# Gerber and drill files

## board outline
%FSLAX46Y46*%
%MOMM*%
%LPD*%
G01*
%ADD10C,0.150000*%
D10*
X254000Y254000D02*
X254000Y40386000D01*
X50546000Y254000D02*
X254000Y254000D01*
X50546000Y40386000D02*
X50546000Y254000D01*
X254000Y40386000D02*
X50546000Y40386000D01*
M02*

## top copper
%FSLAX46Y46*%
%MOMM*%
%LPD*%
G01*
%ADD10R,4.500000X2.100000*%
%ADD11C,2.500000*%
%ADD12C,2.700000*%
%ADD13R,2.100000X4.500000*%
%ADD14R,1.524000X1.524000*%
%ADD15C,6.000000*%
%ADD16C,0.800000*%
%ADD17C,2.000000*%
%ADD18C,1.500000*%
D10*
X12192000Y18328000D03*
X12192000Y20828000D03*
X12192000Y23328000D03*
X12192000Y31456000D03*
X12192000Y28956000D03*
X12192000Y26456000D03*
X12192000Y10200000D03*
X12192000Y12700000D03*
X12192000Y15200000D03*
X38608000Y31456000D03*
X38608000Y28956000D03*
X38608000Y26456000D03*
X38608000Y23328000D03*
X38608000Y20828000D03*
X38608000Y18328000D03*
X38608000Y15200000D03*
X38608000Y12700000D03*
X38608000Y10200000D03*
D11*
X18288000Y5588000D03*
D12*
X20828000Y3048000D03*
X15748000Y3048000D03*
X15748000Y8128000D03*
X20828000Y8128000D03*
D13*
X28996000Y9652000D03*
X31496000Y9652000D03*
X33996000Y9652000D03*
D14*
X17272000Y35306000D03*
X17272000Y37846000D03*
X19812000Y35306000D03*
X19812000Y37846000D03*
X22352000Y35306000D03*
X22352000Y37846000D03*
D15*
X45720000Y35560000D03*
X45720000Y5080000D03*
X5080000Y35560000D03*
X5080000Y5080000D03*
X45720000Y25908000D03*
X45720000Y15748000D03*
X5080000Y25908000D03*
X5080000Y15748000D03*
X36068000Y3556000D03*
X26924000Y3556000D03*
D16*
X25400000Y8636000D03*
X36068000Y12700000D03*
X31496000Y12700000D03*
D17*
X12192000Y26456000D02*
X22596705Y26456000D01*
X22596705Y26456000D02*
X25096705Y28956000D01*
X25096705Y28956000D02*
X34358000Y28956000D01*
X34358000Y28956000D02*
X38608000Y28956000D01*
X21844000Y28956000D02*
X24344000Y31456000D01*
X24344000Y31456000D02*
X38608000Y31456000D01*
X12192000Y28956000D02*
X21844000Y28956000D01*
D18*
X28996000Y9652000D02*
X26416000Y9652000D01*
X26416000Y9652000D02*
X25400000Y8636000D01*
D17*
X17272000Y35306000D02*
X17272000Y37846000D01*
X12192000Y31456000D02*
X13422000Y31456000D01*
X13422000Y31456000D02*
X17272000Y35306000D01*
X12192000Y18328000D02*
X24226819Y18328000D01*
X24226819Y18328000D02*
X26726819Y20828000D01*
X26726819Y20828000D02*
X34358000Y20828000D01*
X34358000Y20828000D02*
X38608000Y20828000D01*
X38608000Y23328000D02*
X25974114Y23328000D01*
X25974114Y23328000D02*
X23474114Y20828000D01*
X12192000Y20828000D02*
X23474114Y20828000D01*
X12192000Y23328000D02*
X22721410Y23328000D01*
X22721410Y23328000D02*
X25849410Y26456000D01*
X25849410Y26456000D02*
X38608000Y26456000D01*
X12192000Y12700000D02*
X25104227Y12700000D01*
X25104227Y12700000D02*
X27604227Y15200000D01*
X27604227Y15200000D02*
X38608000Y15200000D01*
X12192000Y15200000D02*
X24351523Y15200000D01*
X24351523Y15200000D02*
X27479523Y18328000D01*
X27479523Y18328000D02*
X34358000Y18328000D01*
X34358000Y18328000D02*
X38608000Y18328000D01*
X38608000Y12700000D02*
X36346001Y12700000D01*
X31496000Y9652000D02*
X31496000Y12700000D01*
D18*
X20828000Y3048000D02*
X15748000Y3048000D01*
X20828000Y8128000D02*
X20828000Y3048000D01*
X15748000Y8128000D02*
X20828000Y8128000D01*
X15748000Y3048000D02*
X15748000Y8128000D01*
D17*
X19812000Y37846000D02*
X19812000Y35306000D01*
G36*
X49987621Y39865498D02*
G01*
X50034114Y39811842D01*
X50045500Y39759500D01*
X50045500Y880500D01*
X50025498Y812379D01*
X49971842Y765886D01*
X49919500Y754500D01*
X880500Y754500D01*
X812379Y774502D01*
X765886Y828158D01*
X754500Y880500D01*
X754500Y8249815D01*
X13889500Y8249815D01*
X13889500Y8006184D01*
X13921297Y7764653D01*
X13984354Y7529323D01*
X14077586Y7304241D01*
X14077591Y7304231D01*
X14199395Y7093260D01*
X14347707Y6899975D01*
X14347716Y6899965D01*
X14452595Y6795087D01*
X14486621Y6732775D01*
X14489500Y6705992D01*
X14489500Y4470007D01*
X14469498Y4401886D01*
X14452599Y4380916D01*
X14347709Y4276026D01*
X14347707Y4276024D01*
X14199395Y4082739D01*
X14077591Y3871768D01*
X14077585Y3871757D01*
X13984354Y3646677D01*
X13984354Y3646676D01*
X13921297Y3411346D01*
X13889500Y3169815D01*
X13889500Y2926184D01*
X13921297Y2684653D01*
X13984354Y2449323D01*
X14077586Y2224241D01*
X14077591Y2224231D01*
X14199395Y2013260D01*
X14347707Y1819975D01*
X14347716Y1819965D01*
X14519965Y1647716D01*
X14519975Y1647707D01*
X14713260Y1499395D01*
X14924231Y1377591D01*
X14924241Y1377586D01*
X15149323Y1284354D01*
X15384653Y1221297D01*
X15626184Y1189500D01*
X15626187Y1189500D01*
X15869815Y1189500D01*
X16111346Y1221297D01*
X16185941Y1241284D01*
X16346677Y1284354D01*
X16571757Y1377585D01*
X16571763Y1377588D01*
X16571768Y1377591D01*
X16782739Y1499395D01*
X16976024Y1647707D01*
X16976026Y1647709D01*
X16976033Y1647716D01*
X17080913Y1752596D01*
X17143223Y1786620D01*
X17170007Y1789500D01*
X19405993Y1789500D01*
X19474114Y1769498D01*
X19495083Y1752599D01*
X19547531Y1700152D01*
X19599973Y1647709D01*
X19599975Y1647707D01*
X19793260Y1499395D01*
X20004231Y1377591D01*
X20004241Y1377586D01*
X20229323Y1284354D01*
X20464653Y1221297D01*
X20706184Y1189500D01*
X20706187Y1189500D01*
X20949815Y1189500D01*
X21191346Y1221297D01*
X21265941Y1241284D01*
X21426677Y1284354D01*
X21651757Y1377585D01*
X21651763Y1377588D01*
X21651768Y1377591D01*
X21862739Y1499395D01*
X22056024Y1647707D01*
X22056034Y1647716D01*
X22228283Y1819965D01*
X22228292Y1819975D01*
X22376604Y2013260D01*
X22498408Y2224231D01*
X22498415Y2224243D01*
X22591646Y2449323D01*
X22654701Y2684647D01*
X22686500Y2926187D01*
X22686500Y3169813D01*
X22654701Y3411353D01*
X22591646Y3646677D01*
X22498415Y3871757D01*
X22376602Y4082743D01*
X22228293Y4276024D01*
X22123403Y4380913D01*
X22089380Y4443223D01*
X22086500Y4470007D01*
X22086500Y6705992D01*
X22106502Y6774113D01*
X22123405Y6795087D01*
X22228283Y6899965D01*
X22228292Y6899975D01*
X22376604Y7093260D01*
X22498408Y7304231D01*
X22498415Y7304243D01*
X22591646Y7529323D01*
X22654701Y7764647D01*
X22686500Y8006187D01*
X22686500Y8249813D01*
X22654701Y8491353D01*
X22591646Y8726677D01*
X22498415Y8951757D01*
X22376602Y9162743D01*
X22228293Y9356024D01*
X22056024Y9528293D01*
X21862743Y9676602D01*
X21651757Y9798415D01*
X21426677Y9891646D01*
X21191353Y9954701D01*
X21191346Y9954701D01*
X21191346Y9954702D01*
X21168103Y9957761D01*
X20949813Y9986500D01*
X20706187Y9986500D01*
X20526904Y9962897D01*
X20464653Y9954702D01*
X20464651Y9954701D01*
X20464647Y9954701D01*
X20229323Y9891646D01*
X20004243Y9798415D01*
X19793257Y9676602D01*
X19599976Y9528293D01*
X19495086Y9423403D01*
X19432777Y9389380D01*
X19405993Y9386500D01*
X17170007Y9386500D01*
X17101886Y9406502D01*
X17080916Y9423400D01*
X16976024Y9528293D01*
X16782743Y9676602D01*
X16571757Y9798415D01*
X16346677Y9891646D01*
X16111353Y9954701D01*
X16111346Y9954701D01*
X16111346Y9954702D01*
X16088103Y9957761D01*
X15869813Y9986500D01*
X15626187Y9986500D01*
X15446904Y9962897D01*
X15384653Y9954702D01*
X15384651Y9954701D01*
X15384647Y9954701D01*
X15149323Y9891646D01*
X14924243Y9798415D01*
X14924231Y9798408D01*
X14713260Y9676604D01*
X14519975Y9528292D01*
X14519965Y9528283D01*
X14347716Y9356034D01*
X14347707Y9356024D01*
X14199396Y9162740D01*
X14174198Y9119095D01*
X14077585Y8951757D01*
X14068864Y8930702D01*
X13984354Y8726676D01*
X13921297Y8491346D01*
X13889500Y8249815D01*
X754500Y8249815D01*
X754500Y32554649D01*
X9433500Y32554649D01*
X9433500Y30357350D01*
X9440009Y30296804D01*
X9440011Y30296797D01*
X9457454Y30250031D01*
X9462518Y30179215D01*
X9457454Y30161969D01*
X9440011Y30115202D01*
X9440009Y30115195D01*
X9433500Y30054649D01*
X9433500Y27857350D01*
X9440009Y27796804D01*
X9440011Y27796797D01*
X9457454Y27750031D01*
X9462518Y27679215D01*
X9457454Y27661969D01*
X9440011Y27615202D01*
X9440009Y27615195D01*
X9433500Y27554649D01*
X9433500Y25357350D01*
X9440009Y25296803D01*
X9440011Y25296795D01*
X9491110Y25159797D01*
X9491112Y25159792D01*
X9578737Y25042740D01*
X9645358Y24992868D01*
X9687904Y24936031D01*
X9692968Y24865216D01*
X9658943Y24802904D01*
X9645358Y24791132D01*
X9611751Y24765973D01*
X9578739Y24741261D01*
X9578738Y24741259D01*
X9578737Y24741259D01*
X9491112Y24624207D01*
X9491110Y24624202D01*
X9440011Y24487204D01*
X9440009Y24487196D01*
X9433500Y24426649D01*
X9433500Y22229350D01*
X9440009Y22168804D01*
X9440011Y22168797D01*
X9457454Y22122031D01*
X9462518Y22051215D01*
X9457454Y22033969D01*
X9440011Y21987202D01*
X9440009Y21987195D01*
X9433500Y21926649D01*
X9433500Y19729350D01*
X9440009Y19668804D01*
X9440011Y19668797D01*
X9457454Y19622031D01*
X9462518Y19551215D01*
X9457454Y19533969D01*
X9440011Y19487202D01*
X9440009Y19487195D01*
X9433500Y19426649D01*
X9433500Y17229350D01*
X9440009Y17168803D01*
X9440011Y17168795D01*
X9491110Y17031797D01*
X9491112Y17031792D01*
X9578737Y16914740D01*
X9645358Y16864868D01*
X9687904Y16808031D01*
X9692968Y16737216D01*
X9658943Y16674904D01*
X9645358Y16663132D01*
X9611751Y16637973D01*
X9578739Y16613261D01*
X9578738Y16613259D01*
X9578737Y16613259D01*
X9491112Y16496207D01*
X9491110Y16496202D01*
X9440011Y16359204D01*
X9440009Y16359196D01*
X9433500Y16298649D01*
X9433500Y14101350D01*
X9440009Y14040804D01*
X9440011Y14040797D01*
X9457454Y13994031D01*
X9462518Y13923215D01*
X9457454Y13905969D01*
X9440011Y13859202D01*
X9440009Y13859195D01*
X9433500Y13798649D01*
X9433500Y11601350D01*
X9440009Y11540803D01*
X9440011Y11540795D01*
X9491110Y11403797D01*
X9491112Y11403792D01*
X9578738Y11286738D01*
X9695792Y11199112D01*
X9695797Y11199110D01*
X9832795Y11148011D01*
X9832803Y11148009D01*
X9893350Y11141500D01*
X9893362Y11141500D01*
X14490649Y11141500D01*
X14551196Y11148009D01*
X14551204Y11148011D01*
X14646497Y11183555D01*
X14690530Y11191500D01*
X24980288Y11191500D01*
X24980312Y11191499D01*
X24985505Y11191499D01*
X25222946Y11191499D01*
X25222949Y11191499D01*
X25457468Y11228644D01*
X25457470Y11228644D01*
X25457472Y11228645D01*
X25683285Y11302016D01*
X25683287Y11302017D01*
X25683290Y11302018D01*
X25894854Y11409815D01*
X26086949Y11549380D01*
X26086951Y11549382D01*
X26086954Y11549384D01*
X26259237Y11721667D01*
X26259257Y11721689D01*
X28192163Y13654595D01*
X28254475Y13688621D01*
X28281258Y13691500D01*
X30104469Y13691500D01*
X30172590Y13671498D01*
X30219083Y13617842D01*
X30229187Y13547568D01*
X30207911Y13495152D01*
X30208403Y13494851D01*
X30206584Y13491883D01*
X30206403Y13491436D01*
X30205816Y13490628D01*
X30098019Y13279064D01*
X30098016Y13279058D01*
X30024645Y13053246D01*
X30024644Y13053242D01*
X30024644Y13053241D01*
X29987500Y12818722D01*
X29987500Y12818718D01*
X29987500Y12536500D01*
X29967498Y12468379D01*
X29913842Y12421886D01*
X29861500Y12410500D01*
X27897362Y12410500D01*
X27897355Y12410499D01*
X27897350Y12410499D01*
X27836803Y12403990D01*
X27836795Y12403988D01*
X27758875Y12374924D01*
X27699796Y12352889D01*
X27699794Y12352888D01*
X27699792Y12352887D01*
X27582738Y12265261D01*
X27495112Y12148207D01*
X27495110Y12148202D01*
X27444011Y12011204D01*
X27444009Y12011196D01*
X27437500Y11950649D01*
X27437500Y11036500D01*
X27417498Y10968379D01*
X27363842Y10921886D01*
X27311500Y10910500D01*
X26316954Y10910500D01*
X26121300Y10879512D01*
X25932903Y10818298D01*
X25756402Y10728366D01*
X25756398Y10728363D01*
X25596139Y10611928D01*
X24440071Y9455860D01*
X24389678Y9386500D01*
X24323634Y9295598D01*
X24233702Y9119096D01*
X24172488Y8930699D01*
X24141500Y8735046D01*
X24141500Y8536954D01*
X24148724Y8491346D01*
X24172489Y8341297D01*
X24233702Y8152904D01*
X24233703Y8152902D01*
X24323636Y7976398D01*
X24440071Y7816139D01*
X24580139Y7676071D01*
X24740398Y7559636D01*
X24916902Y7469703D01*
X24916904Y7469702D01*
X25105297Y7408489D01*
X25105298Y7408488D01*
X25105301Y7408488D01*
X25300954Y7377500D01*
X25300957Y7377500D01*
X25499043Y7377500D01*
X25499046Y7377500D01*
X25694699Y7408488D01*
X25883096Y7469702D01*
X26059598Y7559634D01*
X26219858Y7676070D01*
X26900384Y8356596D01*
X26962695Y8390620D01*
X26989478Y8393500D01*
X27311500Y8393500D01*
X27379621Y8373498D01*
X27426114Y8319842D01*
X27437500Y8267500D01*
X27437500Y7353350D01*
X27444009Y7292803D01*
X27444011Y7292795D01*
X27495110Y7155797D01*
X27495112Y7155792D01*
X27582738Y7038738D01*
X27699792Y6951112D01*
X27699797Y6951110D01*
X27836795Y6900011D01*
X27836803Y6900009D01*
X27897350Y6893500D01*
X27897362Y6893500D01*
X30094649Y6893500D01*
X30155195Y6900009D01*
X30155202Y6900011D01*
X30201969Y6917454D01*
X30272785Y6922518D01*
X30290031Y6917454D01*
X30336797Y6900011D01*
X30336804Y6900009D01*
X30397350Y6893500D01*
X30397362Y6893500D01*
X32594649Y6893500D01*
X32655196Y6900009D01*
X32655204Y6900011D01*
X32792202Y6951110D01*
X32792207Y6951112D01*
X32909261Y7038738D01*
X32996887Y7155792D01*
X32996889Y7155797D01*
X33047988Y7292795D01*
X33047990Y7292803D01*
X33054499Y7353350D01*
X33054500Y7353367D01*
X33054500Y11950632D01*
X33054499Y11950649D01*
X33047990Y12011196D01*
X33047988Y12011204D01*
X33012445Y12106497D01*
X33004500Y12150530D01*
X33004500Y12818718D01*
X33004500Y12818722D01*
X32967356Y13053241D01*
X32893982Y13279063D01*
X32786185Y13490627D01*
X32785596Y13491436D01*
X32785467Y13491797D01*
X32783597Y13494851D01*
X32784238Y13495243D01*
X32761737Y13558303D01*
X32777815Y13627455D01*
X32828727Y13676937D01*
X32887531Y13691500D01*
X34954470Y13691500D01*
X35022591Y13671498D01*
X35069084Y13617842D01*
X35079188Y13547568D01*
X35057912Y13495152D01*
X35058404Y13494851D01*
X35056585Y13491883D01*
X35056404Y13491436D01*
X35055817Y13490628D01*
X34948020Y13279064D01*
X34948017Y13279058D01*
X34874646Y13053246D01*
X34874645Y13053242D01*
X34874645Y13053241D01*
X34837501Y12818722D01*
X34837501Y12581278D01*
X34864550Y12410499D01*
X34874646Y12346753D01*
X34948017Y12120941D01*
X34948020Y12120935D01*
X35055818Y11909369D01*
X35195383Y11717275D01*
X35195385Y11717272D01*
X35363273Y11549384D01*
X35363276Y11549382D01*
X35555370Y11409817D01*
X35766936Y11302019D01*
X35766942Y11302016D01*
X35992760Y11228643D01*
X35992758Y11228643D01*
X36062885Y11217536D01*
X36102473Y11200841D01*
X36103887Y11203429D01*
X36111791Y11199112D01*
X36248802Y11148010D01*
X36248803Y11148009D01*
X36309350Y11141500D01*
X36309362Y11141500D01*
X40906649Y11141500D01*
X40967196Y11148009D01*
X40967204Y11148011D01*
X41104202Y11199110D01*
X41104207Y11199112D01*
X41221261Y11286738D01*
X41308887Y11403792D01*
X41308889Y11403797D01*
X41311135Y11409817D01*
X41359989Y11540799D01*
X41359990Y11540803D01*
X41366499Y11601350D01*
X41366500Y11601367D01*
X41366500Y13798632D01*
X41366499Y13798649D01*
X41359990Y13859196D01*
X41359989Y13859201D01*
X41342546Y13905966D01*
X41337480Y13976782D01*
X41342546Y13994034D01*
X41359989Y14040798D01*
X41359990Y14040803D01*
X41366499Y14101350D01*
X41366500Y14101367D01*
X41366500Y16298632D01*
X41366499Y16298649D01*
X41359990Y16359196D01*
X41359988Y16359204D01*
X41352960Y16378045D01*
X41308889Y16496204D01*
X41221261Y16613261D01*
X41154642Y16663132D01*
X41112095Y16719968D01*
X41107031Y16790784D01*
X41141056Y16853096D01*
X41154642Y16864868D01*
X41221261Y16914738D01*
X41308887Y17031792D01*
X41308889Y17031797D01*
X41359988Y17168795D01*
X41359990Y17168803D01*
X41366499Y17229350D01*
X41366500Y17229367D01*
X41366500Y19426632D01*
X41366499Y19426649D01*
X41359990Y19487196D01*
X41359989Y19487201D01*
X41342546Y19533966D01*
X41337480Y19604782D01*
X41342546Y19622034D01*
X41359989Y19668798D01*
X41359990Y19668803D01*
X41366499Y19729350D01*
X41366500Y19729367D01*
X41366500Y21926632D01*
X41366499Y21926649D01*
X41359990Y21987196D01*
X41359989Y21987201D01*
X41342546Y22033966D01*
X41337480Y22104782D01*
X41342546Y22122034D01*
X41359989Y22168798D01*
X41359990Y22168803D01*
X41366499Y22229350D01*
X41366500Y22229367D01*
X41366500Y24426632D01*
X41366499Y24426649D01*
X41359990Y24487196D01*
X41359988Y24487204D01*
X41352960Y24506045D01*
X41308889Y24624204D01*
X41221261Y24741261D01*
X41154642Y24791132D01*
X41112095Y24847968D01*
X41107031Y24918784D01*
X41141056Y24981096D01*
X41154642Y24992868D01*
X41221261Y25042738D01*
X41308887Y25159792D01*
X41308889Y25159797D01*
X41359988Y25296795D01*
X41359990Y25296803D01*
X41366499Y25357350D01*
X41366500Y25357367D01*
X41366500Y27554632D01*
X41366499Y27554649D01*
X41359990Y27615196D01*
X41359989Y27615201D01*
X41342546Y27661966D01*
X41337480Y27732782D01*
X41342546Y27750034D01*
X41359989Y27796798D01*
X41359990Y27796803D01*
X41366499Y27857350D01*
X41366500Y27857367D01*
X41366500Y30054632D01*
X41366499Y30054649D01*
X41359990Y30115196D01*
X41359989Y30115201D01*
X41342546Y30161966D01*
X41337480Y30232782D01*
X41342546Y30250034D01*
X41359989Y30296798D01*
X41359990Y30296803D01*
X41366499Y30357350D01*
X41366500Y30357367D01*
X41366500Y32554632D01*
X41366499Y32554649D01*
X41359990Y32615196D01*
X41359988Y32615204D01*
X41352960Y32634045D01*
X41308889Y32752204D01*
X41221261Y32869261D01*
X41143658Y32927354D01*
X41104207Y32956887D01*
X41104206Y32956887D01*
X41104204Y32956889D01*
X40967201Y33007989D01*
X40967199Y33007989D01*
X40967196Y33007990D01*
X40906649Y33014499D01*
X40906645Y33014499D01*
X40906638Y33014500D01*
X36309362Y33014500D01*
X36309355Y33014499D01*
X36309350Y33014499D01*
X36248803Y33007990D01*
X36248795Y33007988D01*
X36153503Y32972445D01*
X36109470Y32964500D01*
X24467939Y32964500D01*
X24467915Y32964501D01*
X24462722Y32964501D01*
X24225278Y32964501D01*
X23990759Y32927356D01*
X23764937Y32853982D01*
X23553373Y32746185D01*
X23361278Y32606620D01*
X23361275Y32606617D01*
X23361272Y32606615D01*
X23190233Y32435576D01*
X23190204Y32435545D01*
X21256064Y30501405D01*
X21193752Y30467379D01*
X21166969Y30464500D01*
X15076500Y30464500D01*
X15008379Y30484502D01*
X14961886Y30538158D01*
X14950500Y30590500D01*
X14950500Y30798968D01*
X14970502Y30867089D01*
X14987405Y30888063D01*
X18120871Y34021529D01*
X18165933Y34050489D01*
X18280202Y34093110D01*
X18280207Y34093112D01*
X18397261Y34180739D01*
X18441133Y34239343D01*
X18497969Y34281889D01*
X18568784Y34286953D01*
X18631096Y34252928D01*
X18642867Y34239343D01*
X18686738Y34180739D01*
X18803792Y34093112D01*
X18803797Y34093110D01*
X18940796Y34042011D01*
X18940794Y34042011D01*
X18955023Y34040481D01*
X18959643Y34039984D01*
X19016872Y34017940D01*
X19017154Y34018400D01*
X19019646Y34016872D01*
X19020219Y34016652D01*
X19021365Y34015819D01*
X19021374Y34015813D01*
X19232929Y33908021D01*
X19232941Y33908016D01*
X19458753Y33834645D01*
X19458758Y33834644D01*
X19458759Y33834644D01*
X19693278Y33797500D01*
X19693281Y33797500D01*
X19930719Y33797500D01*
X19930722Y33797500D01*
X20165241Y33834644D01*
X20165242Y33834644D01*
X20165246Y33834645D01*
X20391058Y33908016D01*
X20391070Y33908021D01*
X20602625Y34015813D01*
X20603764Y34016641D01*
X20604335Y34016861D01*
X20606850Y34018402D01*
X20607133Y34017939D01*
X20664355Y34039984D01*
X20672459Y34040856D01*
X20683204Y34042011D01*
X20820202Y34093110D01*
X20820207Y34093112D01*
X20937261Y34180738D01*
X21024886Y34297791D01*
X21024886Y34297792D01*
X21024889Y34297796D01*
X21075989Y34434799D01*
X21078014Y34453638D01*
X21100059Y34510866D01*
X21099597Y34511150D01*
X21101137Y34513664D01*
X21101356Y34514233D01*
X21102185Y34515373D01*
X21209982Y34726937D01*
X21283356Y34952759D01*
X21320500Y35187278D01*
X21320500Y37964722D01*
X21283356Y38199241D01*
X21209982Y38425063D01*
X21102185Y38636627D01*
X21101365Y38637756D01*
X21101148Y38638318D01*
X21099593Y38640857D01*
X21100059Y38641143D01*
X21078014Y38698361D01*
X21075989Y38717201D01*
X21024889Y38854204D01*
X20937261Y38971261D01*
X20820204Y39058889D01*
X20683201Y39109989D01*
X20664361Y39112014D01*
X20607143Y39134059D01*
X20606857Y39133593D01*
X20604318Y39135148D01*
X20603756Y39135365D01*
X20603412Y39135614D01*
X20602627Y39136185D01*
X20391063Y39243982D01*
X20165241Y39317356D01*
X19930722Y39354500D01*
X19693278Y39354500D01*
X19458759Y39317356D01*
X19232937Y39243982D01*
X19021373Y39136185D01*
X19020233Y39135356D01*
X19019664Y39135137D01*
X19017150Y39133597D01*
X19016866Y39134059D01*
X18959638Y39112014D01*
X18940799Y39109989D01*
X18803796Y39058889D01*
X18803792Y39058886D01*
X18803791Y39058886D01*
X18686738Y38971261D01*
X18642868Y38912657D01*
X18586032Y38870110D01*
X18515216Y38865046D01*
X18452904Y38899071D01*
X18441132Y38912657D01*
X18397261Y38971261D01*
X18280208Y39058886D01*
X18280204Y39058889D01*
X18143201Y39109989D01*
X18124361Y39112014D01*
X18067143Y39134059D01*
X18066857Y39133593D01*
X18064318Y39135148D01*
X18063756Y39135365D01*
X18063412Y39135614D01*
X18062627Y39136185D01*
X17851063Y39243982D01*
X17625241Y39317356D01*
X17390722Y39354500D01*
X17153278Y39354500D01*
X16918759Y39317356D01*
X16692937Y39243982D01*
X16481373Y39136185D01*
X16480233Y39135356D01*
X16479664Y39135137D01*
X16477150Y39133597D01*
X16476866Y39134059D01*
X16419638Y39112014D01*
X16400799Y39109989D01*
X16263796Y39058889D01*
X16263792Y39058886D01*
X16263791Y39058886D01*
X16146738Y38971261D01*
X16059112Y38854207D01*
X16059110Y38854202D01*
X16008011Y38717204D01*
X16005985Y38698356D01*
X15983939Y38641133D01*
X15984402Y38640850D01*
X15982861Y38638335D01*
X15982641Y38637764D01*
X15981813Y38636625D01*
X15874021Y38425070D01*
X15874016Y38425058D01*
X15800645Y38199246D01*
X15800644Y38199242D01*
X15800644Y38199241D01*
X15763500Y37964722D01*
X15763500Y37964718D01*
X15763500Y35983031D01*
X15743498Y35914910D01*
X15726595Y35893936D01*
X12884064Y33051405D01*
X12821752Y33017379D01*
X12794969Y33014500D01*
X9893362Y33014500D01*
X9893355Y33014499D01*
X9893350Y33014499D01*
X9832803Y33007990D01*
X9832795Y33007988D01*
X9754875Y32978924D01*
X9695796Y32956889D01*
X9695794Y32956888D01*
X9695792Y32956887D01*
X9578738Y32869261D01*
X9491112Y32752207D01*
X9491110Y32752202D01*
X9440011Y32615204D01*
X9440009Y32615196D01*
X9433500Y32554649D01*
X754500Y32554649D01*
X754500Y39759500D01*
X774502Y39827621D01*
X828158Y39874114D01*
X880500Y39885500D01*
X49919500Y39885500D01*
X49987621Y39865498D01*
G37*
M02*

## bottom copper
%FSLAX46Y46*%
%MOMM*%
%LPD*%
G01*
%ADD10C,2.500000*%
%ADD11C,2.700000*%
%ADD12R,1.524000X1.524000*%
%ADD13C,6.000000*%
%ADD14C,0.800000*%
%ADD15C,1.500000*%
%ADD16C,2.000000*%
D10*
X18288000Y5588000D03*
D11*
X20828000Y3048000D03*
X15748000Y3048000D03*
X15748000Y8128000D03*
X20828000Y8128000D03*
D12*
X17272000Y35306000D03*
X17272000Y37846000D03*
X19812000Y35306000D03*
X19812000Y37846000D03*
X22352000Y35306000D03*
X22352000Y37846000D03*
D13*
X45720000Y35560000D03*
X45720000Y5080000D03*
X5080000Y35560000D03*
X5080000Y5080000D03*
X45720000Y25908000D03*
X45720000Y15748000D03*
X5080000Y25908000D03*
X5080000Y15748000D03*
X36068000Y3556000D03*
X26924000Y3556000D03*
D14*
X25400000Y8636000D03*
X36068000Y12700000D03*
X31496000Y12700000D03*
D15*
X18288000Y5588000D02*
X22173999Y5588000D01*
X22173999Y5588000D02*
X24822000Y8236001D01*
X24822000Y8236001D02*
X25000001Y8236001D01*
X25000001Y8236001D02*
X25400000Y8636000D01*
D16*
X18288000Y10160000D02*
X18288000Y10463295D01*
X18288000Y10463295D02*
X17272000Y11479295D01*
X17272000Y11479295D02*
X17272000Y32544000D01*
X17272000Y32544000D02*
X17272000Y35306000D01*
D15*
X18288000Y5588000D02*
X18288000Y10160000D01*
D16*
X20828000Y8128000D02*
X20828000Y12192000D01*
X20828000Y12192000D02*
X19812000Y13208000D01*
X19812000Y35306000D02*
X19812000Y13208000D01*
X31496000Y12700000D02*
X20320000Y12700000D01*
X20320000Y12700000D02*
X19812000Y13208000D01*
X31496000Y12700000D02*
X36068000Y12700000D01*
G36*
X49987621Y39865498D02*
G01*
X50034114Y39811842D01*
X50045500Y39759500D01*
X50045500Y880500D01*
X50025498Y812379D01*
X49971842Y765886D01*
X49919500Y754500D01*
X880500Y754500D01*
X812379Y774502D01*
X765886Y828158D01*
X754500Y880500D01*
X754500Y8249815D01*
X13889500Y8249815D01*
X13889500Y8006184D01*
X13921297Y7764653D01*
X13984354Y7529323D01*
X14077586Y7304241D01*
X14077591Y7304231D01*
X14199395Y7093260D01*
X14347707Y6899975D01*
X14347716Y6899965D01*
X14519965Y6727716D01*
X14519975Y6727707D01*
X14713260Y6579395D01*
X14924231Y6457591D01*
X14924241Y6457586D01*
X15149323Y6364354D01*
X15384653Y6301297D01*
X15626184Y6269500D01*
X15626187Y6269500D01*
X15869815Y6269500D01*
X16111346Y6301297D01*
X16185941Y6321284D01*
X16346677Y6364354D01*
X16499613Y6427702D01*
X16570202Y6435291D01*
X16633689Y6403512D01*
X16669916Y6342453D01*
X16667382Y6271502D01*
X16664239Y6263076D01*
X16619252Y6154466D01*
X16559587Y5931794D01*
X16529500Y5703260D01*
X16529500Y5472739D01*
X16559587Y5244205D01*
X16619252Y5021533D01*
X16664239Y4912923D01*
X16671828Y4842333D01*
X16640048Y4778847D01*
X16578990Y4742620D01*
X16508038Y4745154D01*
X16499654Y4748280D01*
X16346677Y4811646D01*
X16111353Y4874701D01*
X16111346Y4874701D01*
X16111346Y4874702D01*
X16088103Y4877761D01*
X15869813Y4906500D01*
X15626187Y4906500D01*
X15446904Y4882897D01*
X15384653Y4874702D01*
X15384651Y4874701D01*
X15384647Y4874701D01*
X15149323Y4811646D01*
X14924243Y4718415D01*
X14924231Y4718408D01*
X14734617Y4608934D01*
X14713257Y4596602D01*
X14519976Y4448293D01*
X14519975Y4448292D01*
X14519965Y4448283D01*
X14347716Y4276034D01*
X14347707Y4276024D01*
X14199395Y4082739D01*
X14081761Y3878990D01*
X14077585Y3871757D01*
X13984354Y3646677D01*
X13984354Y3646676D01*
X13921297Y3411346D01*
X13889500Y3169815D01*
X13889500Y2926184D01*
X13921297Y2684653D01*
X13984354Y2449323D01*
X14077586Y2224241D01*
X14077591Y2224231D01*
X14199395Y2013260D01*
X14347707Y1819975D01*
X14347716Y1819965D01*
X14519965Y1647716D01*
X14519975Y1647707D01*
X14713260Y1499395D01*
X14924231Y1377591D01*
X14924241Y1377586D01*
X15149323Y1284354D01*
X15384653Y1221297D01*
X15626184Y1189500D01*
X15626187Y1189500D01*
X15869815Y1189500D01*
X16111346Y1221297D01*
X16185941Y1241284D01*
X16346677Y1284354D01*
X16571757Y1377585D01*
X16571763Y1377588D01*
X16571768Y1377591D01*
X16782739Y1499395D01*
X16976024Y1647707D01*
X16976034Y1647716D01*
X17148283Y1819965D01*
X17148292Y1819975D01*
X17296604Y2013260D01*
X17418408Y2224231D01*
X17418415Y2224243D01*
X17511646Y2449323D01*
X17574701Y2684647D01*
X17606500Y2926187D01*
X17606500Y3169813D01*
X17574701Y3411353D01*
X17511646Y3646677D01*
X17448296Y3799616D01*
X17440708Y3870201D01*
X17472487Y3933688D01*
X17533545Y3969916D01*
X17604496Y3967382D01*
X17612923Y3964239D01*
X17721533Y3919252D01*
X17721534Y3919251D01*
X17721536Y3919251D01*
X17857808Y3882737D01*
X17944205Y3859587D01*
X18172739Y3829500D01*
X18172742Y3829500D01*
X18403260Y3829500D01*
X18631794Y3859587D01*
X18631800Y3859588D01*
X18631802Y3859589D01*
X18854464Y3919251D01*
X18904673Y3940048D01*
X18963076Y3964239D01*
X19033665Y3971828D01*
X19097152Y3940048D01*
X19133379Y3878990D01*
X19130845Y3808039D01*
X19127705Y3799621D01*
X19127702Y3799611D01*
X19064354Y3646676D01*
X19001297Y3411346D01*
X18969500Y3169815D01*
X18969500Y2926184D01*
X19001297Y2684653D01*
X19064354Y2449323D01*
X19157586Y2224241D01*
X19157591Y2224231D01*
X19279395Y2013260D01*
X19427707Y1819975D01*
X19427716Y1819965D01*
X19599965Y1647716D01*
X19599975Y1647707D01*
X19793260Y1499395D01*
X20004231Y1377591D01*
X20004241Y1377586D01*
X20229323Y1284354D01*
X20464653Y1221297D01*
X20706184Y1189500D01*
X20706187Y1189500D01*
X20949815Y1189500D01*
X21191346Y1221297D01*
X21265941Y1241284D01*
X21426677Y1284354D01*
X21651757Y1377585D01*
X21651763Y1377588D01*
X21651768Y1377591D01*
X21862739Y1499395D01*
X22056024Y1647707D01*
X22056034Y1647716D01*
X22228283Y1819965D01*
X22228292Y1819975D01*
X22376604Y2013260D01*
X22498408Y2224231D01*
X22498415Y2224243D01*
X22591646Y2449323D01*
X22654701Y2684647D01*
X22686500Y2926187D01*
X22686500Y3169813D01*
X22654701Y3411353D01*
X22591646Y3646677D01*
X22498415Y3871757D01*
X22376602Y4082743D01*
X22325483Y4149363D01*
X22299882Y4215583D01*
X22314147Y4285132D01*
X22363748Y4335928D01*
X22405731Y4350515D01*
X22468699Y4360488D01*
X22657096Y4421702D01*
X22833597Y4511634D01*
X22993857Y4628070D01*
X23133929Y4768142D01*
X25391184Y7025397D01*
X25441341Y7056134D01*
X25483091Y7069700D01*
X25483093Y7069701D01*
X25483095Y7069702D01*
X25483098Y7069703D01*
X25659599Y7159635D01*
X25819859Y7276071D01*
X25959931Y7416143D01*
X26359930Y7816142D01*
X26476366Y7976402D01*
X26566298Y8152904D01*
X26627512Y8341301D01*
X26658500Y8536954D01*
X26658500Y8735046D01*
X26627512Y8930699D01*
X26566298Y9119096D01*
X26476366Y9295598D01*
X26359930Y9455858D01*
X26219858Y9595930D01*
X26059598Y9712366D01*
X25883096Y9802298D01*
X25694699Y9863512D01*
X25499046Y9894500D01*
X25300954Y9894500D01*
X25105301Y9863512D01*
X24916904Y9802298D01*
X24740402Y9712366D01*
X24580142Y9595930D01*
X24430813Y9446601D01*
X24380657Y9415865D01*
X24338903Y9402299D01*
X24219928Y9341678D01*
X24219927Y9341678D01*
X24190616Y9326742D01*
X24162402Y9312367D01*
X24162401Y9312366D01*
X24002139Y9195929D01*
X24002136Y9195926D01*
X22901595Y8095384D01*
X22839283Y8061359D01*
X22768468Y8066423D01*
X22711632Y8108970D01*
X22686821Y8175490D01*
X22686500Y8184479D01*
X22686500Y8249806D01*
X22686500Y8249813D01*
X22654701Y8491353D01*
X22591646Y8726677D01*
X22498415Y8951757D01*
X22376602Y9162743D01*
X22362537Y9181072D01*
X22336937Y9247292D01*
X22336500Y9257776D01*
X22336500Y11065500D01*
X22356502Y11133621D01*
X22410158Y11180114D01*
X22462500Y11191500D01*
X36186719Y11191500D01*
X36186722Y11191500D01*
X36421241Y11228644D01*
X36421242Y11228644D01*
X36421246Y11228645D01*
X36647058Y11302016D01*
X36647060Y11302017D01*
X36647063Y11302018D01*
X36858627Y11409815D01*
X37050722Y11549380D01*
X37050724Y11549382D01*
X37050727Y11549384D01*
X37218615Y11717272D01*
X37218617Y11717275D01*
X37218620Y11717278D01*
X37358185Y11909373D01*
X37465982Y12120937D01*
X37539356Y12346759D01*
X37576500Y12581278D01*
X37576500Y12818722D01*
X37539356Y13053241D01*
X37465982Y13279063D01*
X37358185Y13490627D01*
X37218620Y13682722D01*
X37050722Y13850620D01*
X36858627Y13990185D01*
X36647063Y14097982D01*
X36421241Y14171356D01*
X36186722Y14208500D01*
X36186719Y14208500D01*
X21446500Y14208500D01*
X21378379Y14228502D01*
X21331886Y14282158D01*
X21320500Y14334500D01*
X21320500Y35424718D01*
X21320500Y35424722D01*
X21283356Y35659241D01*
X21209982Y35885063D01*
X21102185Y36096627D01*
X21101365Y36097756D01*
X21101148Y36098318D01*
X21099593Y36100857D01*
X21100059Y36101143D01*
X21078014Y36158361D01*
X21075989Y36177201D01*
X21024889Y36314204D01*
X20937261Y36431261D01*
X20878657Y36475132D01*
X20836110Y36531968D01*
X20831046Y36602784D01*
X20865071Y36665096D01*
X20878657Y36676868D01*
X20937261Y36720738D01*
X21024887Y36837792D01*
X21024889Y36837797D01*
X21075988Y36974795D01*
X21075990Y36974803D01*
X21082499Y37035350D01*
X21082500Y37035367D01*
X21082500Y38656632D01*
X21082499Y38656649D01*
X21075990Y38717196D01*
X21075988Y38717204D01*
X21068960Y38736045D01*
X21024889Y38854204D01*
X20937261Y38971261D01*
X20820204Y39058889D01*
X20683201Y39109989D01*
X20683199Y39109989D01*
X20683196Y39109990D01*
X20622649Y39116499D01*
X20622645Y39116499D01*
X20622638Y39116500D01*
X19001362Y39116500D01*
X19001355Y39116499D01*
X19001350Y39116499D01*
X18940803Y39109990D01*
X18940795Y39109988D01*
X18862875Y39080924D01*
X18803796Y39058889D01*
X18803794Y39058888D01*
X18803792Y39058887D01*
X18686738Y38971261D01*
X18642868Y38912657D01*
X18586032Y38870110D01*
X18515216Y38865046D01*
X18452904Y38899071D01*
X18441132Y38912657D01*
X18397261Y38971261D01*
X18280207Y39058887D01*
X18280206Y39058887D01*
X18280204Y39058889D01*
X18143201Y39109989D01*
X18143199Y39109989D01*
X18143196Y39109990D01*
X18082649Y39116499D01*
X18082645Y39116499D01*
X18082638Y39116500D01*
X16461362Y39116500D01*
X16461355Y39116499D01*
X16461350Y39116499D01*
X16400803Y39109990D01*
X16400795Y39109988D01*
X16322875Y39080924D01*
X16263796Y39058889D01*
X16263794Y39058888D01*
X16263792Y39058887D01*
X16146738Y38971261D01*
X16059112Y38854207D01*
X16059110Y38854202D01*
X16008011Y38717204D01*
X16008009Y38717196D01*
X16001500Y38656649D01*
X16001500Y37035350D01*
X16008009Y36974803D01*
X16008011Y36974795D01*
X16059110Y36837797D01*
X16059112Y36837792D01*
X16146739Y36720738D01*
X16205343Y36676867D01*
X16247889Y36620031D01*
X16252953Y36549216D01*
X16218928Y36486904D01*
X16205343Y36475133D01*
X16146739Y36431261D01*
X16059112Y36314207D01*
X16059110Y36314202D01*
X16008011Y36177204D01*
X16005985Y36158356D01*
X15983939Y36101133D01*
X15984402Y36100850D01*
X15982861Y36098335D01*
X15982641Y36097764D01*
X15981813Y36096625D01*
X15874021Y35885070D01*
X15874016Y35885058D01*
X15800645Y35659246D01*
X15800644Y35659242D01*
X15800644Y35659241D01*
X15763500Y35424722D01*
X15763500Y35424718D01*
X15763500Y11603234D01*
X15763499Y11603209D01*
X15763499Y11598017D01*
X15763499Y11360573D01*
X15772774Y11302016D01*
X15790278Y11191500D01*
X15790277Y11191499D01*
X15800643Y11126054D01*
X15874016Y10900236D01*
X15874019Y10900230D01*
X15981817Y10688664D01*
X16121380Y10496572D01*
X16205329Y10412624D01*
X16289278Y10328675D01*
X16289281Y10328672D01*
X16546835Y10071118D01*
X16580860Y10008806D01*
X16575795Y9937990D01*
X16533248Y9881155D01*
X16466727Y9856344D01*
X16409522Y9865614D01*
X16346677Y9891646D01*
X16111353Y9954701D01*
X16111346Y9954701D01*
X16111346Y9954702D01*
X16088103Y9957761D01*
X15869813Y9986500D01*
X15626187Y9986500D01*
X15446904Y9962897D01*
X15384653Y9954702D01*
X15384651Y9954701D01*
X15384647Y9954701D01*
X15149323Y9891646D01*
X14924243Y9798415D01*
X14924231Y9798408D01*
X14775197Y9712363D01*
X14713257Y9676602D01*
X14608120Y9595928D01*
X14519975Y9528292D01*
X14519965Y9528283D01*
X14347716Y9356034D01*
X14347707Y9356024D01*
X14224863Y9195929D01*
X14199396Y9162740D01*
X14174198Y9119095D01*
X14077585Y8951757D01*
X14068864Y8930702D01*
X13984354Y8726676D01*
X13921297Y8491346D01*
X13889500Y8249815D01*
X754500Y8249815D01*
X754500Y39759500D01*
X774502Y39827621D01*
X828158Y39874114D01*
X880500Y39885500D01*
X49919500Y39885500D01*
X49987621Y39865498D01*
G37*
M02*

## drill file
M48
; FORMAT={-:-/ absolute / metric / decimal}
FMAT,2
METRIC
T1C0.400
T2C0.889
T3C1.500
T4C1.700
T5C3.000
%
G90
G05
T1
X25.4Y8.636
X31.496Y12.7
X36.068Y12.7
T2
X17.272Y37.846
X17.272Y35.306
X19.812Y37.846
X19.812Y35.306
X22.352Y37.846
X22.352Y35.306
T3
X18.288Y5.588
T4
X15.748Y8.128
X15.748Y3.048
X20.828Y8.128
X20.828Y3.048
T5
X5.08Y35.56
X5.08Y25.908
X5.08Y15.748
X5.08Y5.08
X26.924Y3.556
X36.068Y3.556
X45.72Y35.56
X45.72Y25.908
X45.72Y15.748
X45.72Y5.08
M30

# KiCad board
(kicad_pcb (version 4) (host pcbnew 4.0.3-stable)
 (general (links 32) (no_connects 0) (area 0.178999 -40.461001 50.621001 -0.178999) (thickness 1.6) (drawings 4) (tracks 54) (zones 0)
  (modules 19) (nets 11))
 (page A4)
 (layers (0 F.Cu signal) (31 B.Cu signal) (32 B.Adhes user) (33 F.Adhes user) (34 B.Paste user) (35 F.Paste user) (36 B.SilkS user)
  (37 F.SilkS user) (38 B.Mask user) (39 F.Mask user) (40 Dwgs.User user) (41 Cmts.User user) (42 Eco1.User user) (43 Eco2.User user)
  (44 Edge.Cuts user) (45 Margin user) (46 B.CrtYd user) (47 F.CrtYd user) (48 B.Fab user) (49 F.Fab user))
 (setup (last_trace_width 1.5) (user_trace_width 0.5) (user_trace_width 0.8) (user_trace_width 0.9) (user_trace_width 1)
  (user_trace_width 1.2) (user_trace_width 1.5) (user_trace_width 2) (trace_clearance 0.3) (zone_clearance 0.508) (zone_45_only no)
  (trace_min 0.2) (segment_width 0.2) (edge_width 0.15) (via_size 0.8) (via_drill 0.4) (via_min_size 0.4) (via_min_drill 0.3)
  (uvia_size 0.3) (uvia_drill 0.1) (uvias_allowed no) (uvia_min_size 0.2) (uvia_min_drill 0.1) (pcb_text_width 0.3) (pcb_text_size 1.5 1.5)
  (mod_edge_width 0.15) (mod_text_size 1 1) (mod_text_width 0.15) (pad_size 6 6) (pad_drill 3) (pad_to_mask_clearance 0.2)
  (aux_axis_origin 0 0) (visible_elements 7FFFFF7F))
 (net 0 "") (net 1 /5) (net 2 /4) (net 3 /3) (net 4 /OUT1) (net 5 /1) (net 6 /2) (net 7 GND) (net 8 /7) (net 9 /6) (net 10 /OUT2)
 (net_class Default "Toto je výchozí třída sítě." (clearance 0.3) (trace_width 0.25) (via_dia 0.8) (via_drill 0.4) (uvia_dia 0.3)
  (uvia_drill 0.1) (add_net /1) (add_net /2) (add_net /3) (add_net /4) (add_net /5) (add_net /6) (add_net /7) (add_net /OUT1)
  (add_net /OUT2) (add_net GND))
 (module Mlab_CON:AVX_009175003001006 (layer F.Cu) (at 12.192 -20.828 90)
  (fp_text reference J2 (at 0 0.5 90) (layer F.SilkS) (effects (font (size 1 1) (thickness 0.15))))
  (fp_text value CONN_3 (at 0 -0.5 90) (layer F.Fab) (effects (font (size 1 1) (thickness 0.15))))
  (pad 1 smd rect (at -2.5 0 90) (size 2.1 4.5) (layers F.Cu F.Paste F.Mask) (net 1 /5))
  (pad 2 smd rect (at 0 0 90) (size 2.1 4.5) (layers F.Cu F.Paste F.Mask) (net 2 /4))
  (pad 3 smd rect (at 2.5 0 90) (size 2.1 4.5) (layers F.Cu F.Paste F.Mask) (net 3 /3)))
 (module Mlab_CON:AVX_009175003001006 (layer F.Cu) (at 12.192 -28.956 270)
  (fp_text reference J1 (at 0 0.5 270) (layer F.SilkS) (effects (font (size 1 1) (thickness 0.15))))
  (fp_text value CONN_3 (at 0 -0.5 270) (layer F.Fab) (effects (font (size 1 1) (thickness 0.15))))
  (pad 1 smd rect (at -2.5 0 270) (size 2.1 4.5) (layers F.Cu F.Paste F.Mask) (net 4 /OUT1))
  (pad 2 smd rect (at 0 0 270) (size 2.1 4.5) (layers F.Cu F.Paste F.Mask) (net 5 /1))
  (pad 3 smd rect (at 2.5 0 270) (size 2.1 4.5) (layers F.Cu F.Paste F.Mask) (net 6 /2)))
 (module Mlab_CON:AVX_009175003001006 (layer F.Cu) (at 12.192 -12.7 90)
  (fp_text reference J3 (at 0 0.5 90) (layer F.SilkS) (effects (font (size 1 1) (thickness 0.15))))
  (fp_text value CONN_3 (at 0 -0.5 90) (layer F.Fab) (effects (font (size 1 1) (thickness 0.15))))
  (pad 1 smd rect (at -2.5 0 90) (size 2.1 4.5) (layers F.Cu F.Paste F.Mask) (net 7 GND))
  (pad 2 smd rect (at 0 0 90) (size 2.1 4.5) (layers F.Cu F.Paste F.Mask) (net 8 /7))
  (pad 3 smd rect (at 2.5 0 90) (size 2.1 4.5) (layers F.Cu F.Paste F.Mask) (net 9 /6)))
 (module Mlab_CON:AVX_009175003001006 (layer F.Cu) (at 38.608 -28.956 270)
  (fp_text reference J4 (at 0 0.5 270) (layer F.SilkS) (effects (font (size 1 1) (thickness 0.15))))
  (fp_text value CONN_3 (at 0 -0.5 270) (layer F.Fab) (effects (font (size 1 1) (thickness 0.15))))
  (pad 1 smd rect (at -2.5 0 270) (size 2.1 4.5) (layers F.Cu F.Paste F.Mask) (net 5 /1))
  (pad 2 smd rect (at 0 0 270) (size 2.1 4.5) (layers F.Cu F.Paste F.Mask) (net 6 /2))
  (pad 3 smd rect (at 2.5 0 270) (size 2.1 4.5) (layers F.Cu F.Paste F.Mask) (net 3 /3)))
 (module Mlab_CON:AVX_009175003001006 (layer F.Cu) (at 38.608 -20.828 270)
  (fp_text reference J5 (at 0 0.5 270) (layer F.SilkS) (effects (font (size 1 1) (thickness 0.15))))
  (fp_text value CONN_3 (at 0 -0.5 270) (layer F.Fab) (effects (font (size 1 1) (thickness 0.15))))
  (pad 1 smd rect (at -2.5 0 270) (size 2.1 4.5) (layers F.Cu F.Paste F.Mask) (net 2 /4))
  (pad 2 smd rect (at 0 0 270) (size 2.1 4.5) (layers F.Cu F.Paste F.Mask) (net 1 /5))
  (pad 3 smd rect (at 2.5 0 270) (size 2.1 4.5) (layers F.Cu F.Paste F.Mask) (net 9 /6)))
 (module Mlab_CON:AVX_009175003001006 (layer F.Cu) (at 38.608 -12.7 270)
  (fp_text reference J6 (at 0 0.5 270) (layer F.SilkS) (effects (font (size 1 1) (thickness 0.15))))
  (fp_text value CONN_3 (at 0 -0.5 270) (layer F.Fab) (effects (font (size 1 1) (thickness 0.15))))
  (pad 1 smd rect (at -2.5 0 270) (size 2.1 4.5) (layers F.Cu F.Paste F.Mask) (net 8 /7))
  (pad 2 smd rect (at 0 0 270) (size 2.1 4.5) (layers F.Cu F.Paste F.Mask) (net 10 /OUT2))
  (pad 3 smd rect (at 2.5 0 270) (size 2.1 4.5) (layers F.Cu F.Paste F.Mask) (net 7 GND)))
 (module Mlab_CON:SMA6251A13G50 (layer F.Cu) (at 18.288 -5.588)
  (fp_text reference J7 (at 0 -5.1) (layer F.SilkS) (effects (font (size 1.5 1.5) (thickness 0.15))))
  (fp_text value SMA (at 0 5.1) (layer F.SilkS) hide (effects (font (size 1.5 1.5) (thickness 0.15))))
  (pad 1 thru_hole circle (at 0 0 180) (size 2.5 2.5) (drill 1.5) (layers *.Cu *.Mask) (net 4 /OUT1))
  (pad 2 thru_hole circle (at 2.54 2.54 180) (size 2.7 2.7) (drill 1.7) (layers *.Cu *.Mask) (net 10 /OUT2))
  (pad 2 thru_hole circle (at -2.54 2.54 180) (size 2.7 2.7) (drill 1.7) (layers *.Cu *.Mask) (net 10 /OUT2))
  (pad 2 thru_hole circle (at -2.54 -2.54 180) (size 2.7 2.7) (drill 1.7) (layers *.Cu *.Mask) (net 10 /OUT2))
  (pad 2 thru_hole circle (at 2.54 -2.54 180) (size 2.7 2.7) (drill 1.7) (layers *.Cu *.Mask) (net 10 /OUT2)))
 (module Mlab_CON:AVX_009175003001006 (layer F.Cu) (at 31.496 -9.652)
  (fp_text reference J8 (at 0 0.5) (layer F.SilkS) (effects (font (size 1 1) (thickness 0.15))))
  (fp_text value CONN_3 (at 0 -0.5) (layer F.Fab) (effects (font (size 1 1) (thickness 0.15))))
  (pad 1 smd rect (at -2.5 0) (size 2.1 4.5) (layers F.Cu F.Paste F.Mask) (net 4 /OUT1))
  (pad 2 smd rect (at 0 0) (size 2.1 4.5) (layers F.Cu F.Paste F.Mask) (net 10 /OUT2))
  (pad 3 smd rect (at 2.5 0) (size 2.1 4.5) (layers F.Cu F.Paste F.Mask) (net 7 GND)))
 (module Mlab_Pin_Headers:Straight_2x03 (layer F.Cu) (at 19.812 -36.576 90)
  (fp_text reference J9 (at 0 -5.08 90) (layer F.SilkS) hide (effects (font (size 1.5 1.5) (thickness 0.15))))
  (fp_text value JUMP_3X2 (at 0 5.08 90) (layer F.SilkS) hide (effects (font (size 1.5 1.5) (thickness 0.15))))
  (pad 1 thru_hole rect (at -1.27 -2.54 90) (size 1.524 1.524) (drill 0.889) (layers *.Cu *.Mask F.SilkS) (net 4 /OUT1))
  (pad 2 thru_hole rect (at 1.27 -2.54 90) (size 1.524 1.524) (drill 0.889) (layers *.Cu *.Mask F.SilkS) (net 4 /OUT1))
  (pad 3 thru_hole rect (at -1.27 0 90) (size 1.524 1.524) (drill 0.889) (layers *.Cu *.Mask F.SilkS) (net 10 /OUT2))
  (pad 4 thru_hole rect (at 1.27 0 90) (size 1.524 1.524) (drill 0.889) (layers *.Cu *.Mask F.SilkS) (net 10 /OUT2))
  (pad 5 thru_hole rect (at -1.27 2.54 90) (size 1.524 1.524) (drill 0.889) (layers *.Cu *.Mask F.SilkS) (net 7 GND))
  (pad 6 thru_hole rect (at 1.27 2.54 90) (size 1.524 1.524) (drill 0.889) (layers *.Cu *.Mask F.SilkS) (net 7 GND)))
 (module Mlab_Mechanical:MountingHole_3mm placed (layer F.Cu) (at 45.72 -35.56)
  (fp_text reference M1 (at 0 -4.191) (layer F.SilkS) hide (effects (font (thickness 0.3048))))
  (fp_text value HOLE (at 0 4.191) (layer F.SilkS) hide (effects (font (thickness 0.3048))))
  (pad 1 thru_hole circle (at 0 0) (size 6 6) (drill 3) (layers *.Cu *.Adhes *.Mask) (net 7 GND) (clearance 1) (zone_connect 2)))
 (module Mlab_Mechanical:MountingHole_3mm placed (layer F.Cu) (at 45.72 -5.08)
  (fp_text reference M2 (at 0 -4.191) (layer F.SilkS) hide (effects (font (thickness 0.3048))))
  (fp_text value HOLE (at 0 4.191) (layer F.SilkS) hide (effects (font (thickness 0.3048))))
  (pad 1 thru_hole circle (at 0 0) (size 6 6) (drill 3) (layers *.Cu *.Adhes *.Mask) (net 7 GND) (clearance 1) (zone_connect 2)))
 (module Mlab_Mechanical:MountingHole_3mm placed (layer F.Cu) (at 5.08 -35.56)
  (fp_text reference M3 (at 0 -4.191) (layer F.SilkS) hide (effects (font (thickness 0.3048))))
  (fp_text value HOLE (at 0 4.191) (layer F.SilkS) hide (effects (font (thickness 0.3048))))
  (pad 1 thru_hole circle (at 0 0) (size 6 6) (drill 3) (layers *.Cu *.Adhes *.Mask) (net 7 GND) (clearance 1) (zone_connect 2)))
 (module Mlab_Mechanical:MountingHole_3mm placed (layer F.Cu) (at 5.08 -5.08)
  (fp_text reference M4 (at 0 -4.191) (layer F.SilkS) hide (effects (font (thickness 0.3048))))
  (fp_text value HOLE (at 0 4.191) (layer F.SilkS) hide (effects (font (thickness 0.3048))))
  (pad 1 thru_hole circle (at 0 0) (size 6 6) (drill 3) (layers *.Cu *.Adhes *.Mask) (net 7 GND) (clearance 1) (zone_connect 2)))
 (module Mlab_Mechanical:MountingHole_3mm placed (layer F.Cu) (at 45.72 -25.908)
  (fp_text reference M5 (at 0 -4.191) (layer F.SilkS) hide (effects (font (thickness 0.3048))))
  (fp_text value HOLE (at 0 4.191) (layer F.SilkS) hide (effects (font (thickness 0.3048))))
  (pad 1 thru_hole circle (at 0 0) (size 6 6) (drill 3) (layers *.Cu *.Adhes *.Mask) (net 7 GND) (clearance 1) (zone_connect 2)))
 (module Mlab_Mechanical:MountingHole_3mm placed (layer F.Cu) (at 45.72 -15.748)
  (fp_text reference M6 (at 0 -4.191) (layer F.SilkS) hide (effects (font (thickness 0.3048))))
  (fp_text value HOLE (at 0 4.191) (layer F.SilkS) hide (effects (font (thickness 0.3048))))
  (pad 1 thru_hole circle (at 0 0) (size 6 6) (drill 3) (layers *.Cu *.Adhes *.Mask) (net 7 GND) (clearance 1) (zone_connect 2)))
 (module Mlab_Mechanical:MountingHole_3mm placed (layer F.Cu) (at 5.08 -25.908)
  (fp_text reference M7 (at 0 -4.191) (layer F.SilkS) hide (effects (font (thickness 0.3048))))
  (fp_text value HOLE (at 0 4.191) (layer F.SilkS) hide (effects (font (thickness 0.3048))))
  (pad 1 thru_hole circle (at 0 0) (size 6 6) (drill 3) (layers *.Cu *.Adhes *.Mask) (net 7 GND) (clearance 1) (zone_connect 2)))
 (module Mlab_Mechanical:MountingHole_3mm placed (layer F.Cu) (at 5.08 -15.748)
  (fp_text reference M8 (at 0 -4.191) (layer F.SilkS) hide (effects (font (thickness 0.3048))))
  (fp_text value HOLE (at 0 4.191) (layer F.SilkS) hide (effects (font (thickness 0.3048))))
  (pad 1 thru_hole circle (at 0 0) (size 6 6) (drill 3) (layers *.Cu *.Adhes *.Mask) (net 7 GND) (clearance 1) (zone_connect 2)))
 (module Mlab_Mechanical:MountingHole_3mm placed (layer F.Cu) (at 36.068 -3.556)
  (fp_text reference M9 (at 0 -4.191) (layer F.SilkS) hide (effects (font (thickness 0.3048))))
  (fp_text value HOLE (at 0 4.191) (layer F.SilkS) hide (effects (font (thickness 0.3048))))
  (pad 1 thru_hole circle (at 0 0) (size 6 6) (drill 3) (layers *.Cu *.Adhes *.Mask) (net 7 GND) (clearance 1) (zone_connect 2)))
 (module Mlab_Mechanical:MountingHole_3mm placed (layer F.Cu) (at 26.924 -3.556)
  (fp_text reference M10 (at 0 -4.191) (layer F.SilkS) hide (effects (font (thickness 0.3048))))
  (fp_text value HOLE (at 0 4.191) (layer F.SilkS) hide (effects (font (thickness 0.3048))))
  (pad 1 thru_hole circle (at 0 0) (size 6 6) (drill 3) (layers *.Cu *.Adhes *.Mask) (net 7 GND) (clearance 1) (zone_connect 2)))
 (gr_line (start 0.254 -0.254) (end 0.254 -40.386) (angle 90) (layer Edge.Cuts) (width 0.15))
 (gr_line (start 50.546 -0.254) (end 0.254 -0.254) (angle 90) (layer Edge.Cuts) (width 0.15))
 (gr_line (start 50.546 -40.386) (end 50.546 -0.254) (angle 90) (layer Edge.Cuts) (width 0.15))
 (gr_line (start 0.254 -40.386) (end 50.546 -40.386) (angle 90) (layer Edge.Cuts) (width 0.15))
 (segment (start 12.192 -26.456) (end 22.596705 -26.456) (width 2) (layer F.Cu) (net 6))
 (segment (start 22.596705 -26.456) (end 25.096705 -28.956) (width 2) (layer F.Cu) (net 6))
 (segment (start 25.096705 -28.956) (end 34.358 -28.956) (width 2) (layer F.Cu) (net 6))
 (segment (start 34.358 -28.956) (end 38.608 -28.956) (width 2) (layer F.Cu) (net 6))
 (segment (start 21.844 -28.956) (end 24.344 -31.456) (width 2) (layer F.Cu) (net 5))
 (segment (start 24.344 -31.456) (end 38.608 -31.456) (width 2) (layer F.Cu) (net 5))
 (segment (start 12.192 -28.956) (end 21.844 -28.956) (width 2) (layer F.Cu) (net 5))
 (segment (start 18.288 -5.588) (end 22.173999 -5.588) (width 1.5) (layer B.Cu) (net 4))
 (segment (start 22.173999 -5.588) (end 24.822 -8.236001) (width 1.5) (layer B.Cu) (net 4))
 (segment (start 24.822 -8.236001) (end 25.000001 -8.236001) (width 1.5) (layer B.Cu) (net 4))
 (segment (start 25.000001 -8.236001) (end 25.4 -8.636) (width 1.5) (layer B.Cu) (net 4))
 (segment (start 28.996 -9.652) (end 26.416 -9.652) (width 1.5) (layer F.Cu) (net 4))
 (segment (start 26.416 -9.652) (end 25.4 -8.636) (width 1.5) (layer F.Cu) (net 4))
 (via (at 25.4 -8.636) (size 0.8) (drill 0.4) (layers F.Cu B.Cu) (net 4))
 (segment (start 18.288 -10.16) (end 18.288 -10.463295) (width 2) (layer B.Cu) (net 4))
 (segment (start 18.288 -10.463295) (end 17.272 -11.479295) (width 2) (layer B.Cu) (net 4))
 (segment (start 17.272 -11.479295) (end 17.272 -32.544) (width 2) (layer B.Cu) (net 4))
 (segment (start 17.272 -32.544) (end 17.272 -35.306) (width 2) (layer B.Cu) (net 4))
 (segment (start 18.288 -5.588) (end 18.288 -10.16) (width 1.5) (layer B.Cu) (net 4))
 (segment (start 17.272 -35.306) (end 17.272 -37.846) (width 2) (layer F.Cu) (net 4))
 (segment (start 12.192 -31.456) (end 13.422 -31.456) (width 2) (layer F.Cu) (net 4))
 (segment (start 13.422 -31.456) (end 17.272 -35.306) (width 2) (layer F.Cu) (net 4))
 (segment (start 12.192 -18.328) (end 24.226819 -18.328) (width 2) (layer F.Cu) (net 1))
 (segment (start 24.226819 -18.328) (end 26.726819 -20.828) (width 2) (layer F.Cu) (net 1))
 (segment (start 26.726819 -20.828) (end 34.358 -20.828) (width 2) (layer F.Cu) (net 1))
 (segment (start 34.358 -20.828) (end 38.608 -20.828) (width 2) (layer F.Cu) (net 1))
 (segment (start 38.608 -23.328) (end 25.974114 -23.328) (width 2) (layer F.Cu) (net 2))
 (segment (start 25.974114 -23.328) (end 23.474114 -20.828) (width 2) (layer F.Cu) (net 2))
 (segment (start 12.192 -20.828) (end 23.474114 -20.828) (width 2) (layer F.Cu) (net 2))
 (segment (start 12.192 -23.328) (end 22.72141 -23.328) (width 2) (layer F.Cu) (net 3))
 (segment (start 22.72141 -23.328) (end 25.84941 -26.456) (width 2) (layer F.Cu) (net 3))
 (segment (start 25.84941 -26.456) (end 38.608 -26.456) (width 2) (layer F.Cu) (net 3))
 (segment (start 12.192 -12.7) (end 25.104227 -12.7) (width 2) (layer F.Cu) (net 8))
 (segment (start 25.104227 -12.7) (end 27.604227 -15.2) (width 2) (layer F.Cu) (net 8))
 (segment (start 27.604227 -15.2) (end 38.608 -15.2) (width 2) (layer F.Cu) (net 8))
 (segment (start 12.192 -15.2) (end 24.351523 -15.2) (width 2) (layer F.Cu) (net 9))
 (segment (start 24.351523 -15.2) (end 27.479523 -18.328) (width 2) (layer F.Cu) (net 9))
 (segment (start 27.479523 -18.328) (end 34.358 -18.328) (width 2) (layer F.Cu) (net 9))
 (segment (start 34.358 -18.328) (end 38.608 -18.328) (width 2) (layer F.Cu) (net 9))
 (segment (start 20.828 -8.128) (end 20.828 -12.192) (width 2) (layer B.Cu) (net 10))
 (segment (start 20.828 -12.192) (end 19.812 -13.208) (width 2) (layer B.Cu) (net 10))
 (segment (start 19.812 -35.306) (end 19.812 -13.208) (width 2) (layer B.Cu) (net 10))
 (segment (start 31.496 -12.7) (end 20.32 -12.7) (width 2) (layer B.Cu) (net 10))
 (segment (start 20.32 -12.7) (end 19.812 -13.208) (width 2) (layer B.Cu) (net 10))
 (segment (start 38.608 -12.7) (end 36.346001 -12.7) (width 2) (layer F.Cu) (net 10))
 (segment (start 31.496 -12.7) (end 36.068 -12.7) (width 2) (layer B.Cu) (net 10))
 (via (at 36.068 -12.7) (size 0.8) (drill 0.4) (layers F.Cu B.Cu) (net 10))
 (segment (start 31.496 -9.652) (end 31.496 -12.7) (width 2) (layer F.Cu) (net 10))
 (via (at 31.496 -12.7) (size 0.8) (drill 0.4) (layers F.Cu B.Cu) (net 10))
 (segment (start 20.828 -3.048) (end 15.748 -3.048) (width 1.5) (layer F.Cu) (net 10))
 (segment (start 20.828 -8.128) (end 20.828 -3.048) (width 1.5) (layer F.Cu) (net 10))
 (segment (start 15.748 -8.128) (end 20.828 -8.128) (width 1.5) (layer F.Cu) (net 10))
 (segment (start 15.748 -3.048) (end 15.748 -8.128) (width 1.5) (layer F.Cu) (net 10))
 (segment (start 19.812 -37.846) (end 19.812 -35.306) (width 2) (layer F.Cu) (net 10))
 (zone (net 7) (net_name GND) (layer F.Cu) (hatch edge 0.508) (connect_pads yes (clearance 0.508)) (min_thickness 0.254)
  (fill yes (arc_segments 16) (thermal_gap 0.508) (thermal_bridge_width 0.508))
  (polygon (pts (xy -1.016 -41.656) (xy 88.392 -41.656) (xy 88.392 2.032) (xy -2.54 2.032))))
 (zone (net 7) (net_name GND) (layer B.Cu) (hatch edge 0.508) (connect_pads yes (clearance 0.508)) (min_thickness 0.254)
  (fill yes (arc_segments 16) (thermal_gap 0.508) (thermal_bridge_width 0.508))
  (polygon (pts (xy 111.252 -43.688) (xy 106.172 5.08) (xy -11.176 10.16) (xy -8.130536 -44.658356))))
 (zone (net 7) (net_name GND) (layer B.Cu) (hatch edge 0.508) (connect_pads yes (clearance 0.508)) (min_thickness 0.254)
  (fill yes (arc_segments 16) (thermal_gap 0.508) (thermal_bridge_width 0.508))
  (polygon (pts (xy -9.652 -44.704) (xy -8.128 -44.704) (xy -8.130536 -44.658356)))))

